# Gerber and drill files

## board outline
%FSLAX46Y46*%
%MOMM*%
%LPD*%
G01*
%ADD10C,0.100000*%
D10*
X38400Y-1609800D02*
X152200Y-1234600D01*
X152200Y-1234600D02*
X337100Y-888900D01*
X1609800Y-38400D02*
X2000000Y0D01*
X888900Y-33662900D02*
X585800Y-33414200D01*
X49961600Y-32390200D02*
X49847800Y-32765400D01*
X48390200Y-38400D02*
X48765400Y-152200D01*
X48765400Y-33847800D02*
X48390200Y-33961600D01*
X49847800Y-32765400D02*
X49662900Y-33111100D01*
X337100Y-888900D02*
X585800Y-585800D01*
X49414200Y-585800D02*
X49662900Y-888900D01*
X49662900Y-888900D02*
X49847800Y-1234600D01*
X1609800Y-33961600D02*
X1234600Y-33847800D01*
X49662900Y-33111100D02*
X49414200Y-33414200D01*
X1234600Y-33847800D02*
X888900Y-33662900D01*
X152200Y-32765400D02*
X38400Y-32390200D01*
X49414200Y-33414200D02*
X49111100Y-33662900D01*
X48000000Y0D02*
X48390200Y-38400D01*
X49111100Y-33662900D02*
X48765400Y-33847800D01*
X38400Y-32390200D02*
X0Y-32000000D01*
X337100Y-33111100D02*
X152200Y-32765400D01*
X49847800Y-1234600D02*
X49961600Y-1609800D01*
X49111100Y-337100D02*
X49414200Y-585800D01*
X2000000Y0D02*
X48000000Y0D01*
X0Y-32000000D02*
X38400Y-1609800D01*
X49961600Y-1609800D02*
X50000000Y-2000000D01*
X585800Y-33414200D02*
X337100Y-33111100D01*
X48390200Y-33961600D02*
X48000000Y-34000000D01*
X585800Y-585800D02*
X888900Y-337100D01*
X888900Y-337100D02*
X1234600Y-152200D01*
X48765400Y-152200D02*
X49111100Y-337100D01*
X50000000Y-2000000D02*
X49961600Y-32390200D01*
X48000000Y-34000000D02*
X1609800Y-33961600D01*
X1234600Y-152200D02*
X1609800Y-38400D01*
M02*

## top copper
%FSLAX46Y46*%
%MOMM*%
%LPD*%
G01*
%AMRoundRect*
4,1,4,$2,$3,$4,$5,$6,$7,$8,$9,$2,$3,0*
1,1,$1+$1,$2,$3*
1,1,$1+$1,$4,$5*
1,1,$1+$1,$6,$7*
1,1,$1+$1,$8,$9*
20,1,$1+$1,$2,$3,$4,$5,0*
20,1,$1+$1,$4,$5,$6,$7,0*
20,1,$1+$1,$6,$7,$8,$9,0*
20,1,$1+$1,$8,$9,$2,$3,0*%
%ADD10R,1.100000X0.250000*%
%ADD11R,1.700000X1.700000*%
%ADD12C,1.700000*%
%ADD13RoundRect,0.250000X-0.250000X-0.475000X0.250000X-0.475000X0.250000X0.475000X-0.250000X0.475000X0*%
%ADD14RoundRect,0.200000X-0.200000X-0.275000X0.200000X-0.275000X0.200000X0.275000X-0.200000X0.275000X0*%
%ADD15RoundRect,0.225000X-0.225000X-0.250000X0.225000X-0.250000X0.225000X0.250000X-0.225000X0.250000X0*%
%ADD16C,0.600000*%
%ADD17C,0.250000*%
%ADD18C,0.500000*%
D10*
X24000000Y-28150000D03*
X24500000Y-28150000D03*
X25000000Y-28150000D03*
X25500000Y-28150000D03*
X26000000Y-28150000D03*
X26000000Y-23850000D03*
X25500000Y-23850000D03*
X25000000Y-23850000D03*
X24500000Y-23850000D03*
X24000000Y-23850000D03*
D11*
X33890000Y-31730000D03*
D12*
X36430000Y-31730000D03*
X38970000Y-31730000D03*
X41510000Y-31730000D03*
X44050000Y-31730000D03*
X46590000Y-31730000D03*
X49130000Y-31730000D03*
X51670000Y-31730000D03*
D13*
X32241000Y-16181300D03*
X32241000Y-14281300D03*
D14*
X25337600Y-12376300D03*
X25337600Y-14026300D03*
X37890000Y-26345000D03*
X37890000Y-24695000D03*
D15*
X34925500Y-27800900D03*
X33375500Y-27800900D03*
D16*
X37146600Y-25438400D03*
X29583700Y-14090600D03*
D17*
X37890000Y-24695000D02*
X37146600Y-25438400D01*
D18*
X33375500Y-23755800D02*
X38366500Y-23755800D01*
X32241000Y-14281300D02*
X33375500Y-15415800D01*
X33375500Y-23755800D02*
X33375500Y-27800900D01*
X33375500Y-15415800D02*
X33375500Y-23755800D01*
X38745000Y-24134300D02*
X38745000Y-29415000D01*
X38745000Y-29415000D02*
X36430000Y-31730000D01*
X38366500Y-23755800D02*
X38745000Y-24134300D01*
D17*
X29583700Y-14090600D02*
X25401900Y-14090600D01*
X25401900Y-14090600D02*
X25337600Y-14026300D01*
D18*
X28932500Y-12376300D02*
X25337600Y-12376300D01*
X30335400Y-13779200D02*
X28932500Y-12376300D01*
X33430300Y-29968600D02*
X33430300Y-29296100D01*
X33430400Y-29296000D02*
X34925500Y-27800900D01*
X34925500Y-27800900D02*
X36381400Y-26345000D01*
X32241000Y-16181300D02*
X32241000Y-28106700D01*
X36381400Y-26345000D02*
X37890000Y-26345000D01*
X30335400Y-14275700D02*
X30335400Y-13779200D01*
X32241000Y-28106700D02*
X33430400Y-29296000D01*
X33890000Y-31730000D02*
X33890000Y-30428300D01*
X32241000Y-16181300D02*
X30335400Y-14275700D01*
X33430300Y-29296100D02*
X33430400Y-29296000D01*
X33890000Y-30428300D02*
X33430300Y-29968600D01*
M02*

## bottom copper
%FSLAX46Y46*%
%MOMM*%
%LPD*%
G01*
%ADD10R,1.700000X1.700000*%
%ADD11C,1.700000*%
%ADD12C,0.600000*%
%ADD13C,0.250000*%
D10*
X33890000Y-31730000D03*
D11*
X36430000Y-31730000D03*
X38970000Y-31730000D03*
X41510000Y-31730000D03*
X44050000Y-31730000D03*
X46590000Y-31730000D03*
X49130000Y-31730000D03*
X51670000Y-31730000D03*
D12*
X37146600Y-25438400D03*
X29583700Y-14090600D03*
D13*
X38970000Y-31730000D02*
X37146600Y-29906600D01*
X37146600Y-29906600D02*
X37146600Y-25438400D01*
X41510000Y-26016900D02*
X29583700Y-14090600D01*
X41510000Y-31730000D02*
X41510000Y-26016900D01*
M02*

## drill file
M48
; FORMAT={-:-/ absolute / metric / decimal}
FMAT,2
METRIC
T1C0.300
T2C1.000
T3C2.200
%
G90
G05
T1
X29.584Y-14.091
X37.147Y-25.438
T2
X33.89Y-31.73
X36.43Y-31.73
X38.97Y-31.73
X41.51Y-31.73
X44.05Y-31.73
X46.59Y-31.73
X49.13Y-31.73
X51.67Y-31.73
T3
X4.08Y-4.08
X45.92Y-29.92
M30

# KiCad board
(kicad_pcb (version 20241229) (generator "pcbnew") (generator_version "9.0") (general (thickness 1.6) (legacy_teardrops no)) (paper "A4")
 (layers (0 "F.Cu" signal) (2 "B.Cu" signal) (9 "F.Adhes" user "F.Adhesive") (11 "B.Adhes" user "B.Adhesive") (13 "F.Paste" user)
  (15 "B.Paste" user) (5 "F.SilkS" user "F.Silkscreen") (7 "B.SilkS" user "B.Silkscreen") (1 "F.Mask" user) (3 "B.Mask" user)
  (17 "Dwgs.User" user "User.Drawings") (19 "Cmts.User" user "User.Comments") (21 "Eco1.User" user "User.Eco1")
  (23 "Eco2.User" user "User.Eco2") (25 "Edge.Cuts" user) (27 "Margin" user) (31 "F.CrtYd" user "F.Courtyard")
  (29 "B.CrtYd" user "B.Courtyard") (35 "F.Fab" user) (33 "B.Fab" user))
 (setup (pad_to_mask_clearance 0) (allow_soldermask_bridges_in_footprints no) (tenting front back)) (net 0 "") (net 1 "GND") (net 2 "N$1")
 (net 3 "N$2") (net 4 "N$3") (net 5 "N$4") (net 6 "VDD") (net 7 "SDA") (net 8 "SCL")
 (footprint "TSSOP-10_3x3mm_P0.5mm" (layer "F.Cu") (at 25 26 90)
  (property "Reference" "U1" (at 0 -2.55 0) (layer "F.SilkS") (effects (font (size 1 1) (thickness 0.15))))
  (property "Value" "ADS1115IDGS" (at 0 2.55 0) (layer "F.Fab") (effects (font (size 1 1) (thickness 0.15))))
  (pad "1" smd rect (at -2.15 -1) (size 1.1 0.25) (layers "F.Cu" "F.Mask" "F.Paste") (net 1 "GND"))
  (pad "2" smd rect (at -2.15 -0.5) (size 1.1 0.25) (layers "F.Cu" "F.Mask" "F.Paste"))
  (pad "3" smd rect (at -2.15 0) (size 1.1 0.25) (layers "F.Cu" "F.Mask" "F.Paste") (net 1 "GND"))
  (pad "4" smd rect (at -2.15 0.5) (size 1.1 0.25) (layers "F.Cu" "F.Mask" "F.Paste") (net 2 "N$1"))
  (pad "5" smd rect (at -2.15 1) (size 1.1 0.25) (layers "F.Cu" "F.Mask" "F.Paste") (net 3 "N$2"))
  (pad "6" smd rect (at 2.15 1) (size 1.1 0.25) (layers "F.Cu" "F.Mask" "F.Paste") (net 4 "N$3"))
  (pad "7" smd rect (at 2.15 0.5) (size 1.1 0.25) (layers "F.Cu" "F.Mask" "F.Paste") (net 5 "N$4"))
  (pad "8" smd rect (at 2.15 0) (size 1.1 0.25) (layers "F.Cu" "F.Mask" "F.Paste") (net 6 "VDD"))
  (pad "9" smd rect (at 2.15 -0.5) (size 1.1 0.25) (layers "F.Cu" "F.Mask" "F.Paste") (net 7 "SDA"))
  (pad "10" smd rect (at 2.15 -1) (size 1.1 0.25) (layers "F.Cu" "F.Mask" "F.Paste") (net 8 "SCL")))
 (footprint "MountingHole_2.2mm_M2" (layer "F.Cu") (at 4.08 4.08)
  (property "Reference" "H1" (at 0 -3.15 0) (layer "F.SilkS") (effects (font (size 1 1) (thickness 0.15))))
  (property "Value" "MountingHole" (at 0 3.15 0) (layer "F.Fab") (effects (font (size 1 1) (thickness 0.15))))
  (pad "" np_thru_hole circle (at 0 0) (size 2.2 2.2) (drill 2.2) (layers "*.Cu" "*.Mask")))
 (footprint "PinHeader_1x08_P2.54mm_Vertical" (layer "F.Cu") (at 33.89 31.73 90)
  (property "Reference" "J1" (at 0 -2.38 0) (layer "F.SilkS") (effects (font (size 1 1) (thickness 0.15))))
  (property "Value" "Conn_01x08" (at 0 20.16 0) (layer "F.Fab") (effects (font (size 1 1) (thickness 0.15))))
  (pad "1" thru_hole rect (at 0 0) (size 1.7 1.7) (drill 1) (layers "*.Cu" "*.Mask") (remove_unused_layers no) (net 6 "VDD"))
  (pad "2" thru_hole circle (at 0 2.54) (size 1.7 1.7) (drill 1) (layers "*.Cu" "*.Mask") (remove_unused_layers no) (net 1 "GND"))
  (pad "3" thru_hole circle (at 0 5.08) (size 1.7 1.7) (drill 1) (layers "*.Cu" "*.Mask") (remove_unused_layers no) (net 7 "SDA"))
  (pad "4" thru_hole circle (at 0 7.62) (size 1.7 1.7) (drill 1) (layers "*.Cu" "*.Mask") (remove_unused_layers no) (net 8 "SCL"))
  (pad "5" thru_hole circle (at 0 10.16) (size 1.7 1.7) (drill 1) (layers "*.Cu" "*.Mask") (remove_unused_layers no) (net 2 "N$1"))
  (pad "6" thru_hole circle (at 0 12.7) (size 1.7 1.7) (drill 1) (layers "*.Cu" "*.Mask") (remove_unused_layers no) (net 3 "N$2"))
  (pad "7" thru_hole circle (at 0 15.24) (size 1.7 1.7) (drill 1) (layers "*.Cu" "*.Mask") (remove_unused_layers no) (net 4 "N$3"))
  (pad "8" thru_hole circle (at 0 17.78) (size 1.7 1.7) (drill 1) (layers "*.Cu" "*.Mask") (remove_unused_layers no) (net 5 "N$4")))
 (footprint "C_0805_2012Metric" (layer "F.Cu") (at 32.241 15.2313 90)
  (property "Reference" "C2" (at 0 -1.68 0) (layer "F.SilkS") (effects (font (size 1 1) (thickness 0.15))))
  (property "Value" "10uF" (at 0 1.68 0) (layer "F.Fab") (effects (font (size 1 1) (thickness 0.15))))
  (pad "1" smd roundrect (at -0.95 0) (size 1 1.45) (layers "F.Cu" "F.Mask" "F.Paste") (roundrect_rratio 0.25) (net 6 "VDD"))
  (pad "2" smd roundrect (at 0.95 0) (size 1 1.45) (layers "F.Cu" "F.Mask" "F.Paste") (roundrect_rratio 0.25) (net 1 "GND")))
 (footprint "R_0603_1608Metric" (layer "F.Cu") (at 25.3376 13.2013 -90)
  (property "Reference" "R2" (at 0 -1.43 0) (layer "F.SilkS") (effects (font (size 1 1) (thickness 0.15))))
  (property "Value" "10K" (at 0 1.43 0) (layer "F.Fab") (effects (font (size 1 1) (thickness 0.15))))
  (pad "1" smd roundrect (at -0.825 0) (size 0.8 0.95) (layers "F.Cu" "F.Mask" "F.Paste") (roundrect_rratio 0.25) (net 6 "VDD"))
  (pad "2" smd roundrect (at 0.825 0) (size 0.8 0.95) (layers "F.Cu" "F.Mask" "F.Paste") (roundrect_rratio 0.25) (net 8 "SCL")))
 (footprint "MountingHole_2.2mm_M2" (layer "F.Cu") (at 45.92 29.92)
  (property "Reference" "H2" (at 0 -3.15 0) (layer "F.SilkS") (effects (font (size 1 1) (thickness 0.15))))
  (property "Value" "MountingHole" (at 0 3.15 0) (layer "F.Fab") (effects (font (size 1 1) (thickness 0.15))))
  (pad "" np_thru_hole circle (at 0 0) (size 2.2 2.2) (drill 2.2) (layers "*.Cu" "*.Mask")))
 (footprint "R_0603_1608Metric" (layer "F.Cu") (at 37.89 25.52 90)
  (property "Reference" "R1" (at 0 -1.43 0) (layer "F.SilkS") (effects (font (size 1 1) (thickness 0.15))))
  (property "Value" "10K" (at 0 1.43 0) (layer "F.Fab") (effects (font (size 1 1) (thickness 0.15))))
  (pad "1" smd roundrect (at -0.825 0) (size 0.8 0.95) (layers "F.Cu" "F.Mask" "F.Paste") (roundrect_rratio 0.25) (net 6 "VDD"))
  (pad "2" smd roundrect (at 0.825 0) (size 0.8 0.95) (layers "F.Cu" "F.Mask" "F.Paste") (roundrect_rratio 0.25) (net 7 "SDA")))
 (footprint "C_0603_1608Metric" (layer "F.Cu") (at 34.1505 27.8009 180)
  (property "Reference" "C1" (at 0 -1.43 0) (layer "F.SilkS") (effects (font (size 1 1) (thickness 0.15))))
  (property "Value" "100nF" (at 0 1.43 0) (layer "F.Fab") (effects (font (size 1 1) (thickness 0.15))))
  (pad "1" smd roundrect (at -0.775 0) (size 0.9 0.95) (layers "F.Cu" "F.Mask" "F.Paste") (roundrect_rratio 0.25) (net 6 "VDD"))
  (pad "2" smd roundrect (at 0.775 0) (size 0.9 0.95) (layers "F.Cu" "F.Mask" "F.Paste") (roundrect_rratio 0.25) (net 1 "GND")))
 (gr_line (start 0.0384 1.6098) (end 0.1522 1.2346) (stroke (width 0.1) (type solid)) (layer "Edge.Cuts"))
 (gr_line (start 0.1522 1.2346) (end 0.3371 0.8889) (stroke (width 0.1) (type solid)) (layer "Edge.Cuts"))
 (gr_line (start 1.6098 0.0384) (end 2 0) (stroke (width 0.1) (type solid)) (layer "Edge.Cuts"))
 (gr_line (start 0.8889 33.6629) (end 0.5858 33.4142) (stroke (width 0.1) (type solid)) (layer "Edge.Cuts"))
 (gr_line (start 49.9616 32.3902) (end 49.8478 32.7654) (stroke (width 0.1) (type solid)) (layer "Edge.Cuts"))
 (gr_line (start 48.3902 0.0384) (end 48.7654 0.1522) (stroke (width 0.1) (type solid)) (layer "Edge.Cuts"))
 (gr_line (start 48.7654 33.8478) (end 48.3902 33.9616) (stroke (width 0.1) (type solid)) (layer "Edge.Cuts"))
 (gr_line (start 49.8478 32.7654) (end 49.6629 33.1111) (stroke (width 0.1) (type solid)) (layer "Edge.Cuts"))
 (gr_line (start 0.3371 0.8889) (end 0.5858 0.5858) (stroke (width 0.1) (type solid)) (layer "Edge.Cuts"))
 (gr_line (start 49.4142 0.5858) (end 49.6629 0.8889) (stroke (width 0.1) (type solid)) (layer "Edge.Cuts"))
 (gr_line (start 49.6629 0.8889) (end 49.8478 1.2346) (stroke (width 0.1) (type solid)) (layer "Edge.Cuts"))
 (gr_line (start 1.6098 33.9616) (end 1.2346 33.8478) (stroke (width 0.1) (type solid)) (layer "Edge.Cuts"))
 (gr_line (start 49.6629 33.1111) (end 49.4142 33.4142) (stroke (width 0.1) (type solid)) (layer "Edge.Cuts"))
 (gr_line (start 1.2346 33.8478) (end 0.8889 33.6629) (stroke (width 0.1) (type solid)) (layer "Edge.Cuts"))
 (gr_line (start 0.1522 32.7654) (end 0.0384 32.3902) (stroke (width 0.1) (type solid)) (layer "Edge.Cuts"))
 (gr_line (start 49.4142 33.4142) (end 49.1111 33.6629) (stroke (width 0.1) (type solid)) (layer "Edge.Cuts"))
 (gr_line (start 48 0) (end 48.3902 0.0384) (stroke (width 0.1) (type solid)) (layer "Edge.Cuts"))
 (gr_line (start 49.1111 33.6629) (end 48.7654 33.8478) (stroke (width 0.1) (type solid)) (layer "Edge.Cuts"))
 (gr_line (start 0.0384 32.3902) (end 0 32) (stroke (width 0.1) (type solid)) (layer "Edge.Cuts"))
 (gr_line (start 0.3371 33.1111) (end 0.1522 32.7654) (stroke (width 0.1) (type solid)) (layer "Edge.Cuts"))
 (gr_line (start 49.8478 1.2346) (end 49.9616 1.6098) (stroke (width 0.1) (type solid)) (layer "Edge.Cuts"))
 (gr_line (start 49.1111 0.3371) (end 49.4142 0.5858) (stroke (width 0.1) (type solid)) (layer "Edge.Cuts"))
 (gr_line (start 2 0) (end 48 0) (stroke (width 0.1) (type solid)) (layer "Edge.Cuts"))
 (gr_line (start 0 32) (end 0.0384 1.6098) (stroke (width 0.1) (type solid)) (layer "Edge.Cuts"))
 (gr_line (start 49.9616 1.6098) (end 50 2) (stroke (width 0.1) (type solid)) (layer "Edge.Cuts"))
 (gr_line (start 0.5858 33.4142) (end 0.3371 33.1111) (stroke (width 0.1) (type solid)) (layer "Edge.Cuts"))
 (gr_line (start 48.3902 33.9616) (end 48 34) (stroke (width 0.1) (type solid)) (layer "Edge.Cuts"))
 (gr_line (start 0.5858 0.5858) (end 0.8889 0.3371) (stroke (width 0.1) (type solid)) (layer "Edge.Cuts"))
 (gr_line (start 0.8889 0.3371) (end 1.2346 0.1522) (stroke (width 0.1) (type solid)) (layer "Edge.Cuts"))
 (gr_line (start 48.7654 0.1522) (end 49.1111 0.3371) (stroke (width 0.1) (type solid)) (layer "Edge.Cuts"))
 (gr_line (start 50 2) (end 49.9616 32.3902) (stroke (width 0.1) (type solid)) (layer "Edge.Cuts"))
 (gr_line (start 48 34) (end 1.6098 33.9616) (stroke (width 0.1) (type solid)) (layer "Edge.Cuts"))
 (gr_line (start 1.2346 0.1522) (end 1.6098 0.0384) (stroke (width 0.1) (type solid)) (layer "Edge.Cuts"))
 (segment (start 37.89 24.695) (end 37.1466 25.4384) (width 0.25) (layer "F.Cu") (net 7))
 (via (at 37.1466 25.4384) (size 0.6) (drill 0.3) (layers "F.Cu" "B.Cu") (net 7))
 (segment (start 38.97 31.73) (end 37.1466 29.9066) (width 0.25) (layer "B.Cu") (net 7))
 (segment (start 37.1466 29.9066) (end 37.1466 25.4384) (width 0.25) (layer "B.Cu") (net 7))
 (segment (start 33.3755 23.7558) (end 38.3665 23.7558) (width 0.5) (layer "F.Cu") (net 1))
 (segment (start 32.241 14.2813) (end 33.3755 15.4158) (width 0.5) (layer "F.Cu") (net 1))
 (segment (start 33.3755 23.7558) (end 33.3755 27.8009) (width 0.5) (layer "F.Cu") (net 1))
 (segment (start 33.3755 15.4158) (end 33.3755 23.7558) (width 0.5) (layer "F.Cu") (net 1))
 (segment (start 38.745 24.1343) (end 38.745 29.415) (width 0.5) (layer "F.Cu") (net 1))
 (segment (start 38.745 29.415) (end 36.43 31.73) (width 0.5) (layer "F.Cu") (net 1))
 (segment (start 38.3665 23.7558) (end 38.745 24.1343) (width 0.5) (layer "F.Cu") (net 1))
 (segment (start 29.5837 14.0906) (end 25.4019 14.0906) (width 0.25) (layer "F.Cu") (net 8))
 (segment (start 25.4019 14.0906) (end 25.3376 14.0263) (width 0.25) (layer "F.Cu") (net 8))
 (via (at 29.5837 14.0906) (size 0.6) (drill 0.3) (layers "F.Cu" "B.Cu") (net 8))
 (segment (start 41.51 26.0169) (end 29.5837 14.0906) (width 0.25) (layer "B.Cu") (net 8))
 (segment (start 41.51 31.73) (end 41.51 26.0169) (width 0.25) (layer "B.Cu") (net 8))
 (segment (start 28.9325 12.3763) (end 25.3376 12.3763) (width 0.5) (layer "F.Cu") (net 6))
 (segment (start 30.3354 13.7792) (end 28.9325 12.3763) (width 0.5) (layer "F.Cu") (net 6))
 (segment (start 33.4303 29.9686) (end 33.4303 29.2961) (width 0.5) (layer "F.Cu") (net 6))
 (segment (start 33.4304 29.296) (end 34.9255 27.8009) (width 0.5) (layer "F.Cu") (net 6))
 (segment (start 34.9255 27.8009) (end 36.3814 26.345) (width 0.5) (layer "F.Cu") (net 6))
 (segment (start 32.241 16.1813) (end 32.241 28.1067) (width 0.5) (layer "F.Cu") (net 6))
 (segment (start 36.3814 26.345) (end 37.89 26.345) (width 0.5) (layer "F.Cu") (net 6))
 (segment (start 30.3354 14.2757) (end 30.3354 13.7792) (width 0.5) (layer "F.Cu") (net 6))
 (segment (start 32.241 28.1067) (end 33.4304 29.296) (width 0.5) (layer "F.Cu") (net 6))
 (segment (start 33.89 31.73) (end 33.89 30.4283) (width 0.5) (layer "F.Cu") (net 6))
 (segment (start 32.241 16.1813) (end 30.3354 14.2757) (width 0.5) (layer "F.Cu") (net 6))
 (segment (start 33.4303 29.2961) (end 33.4304 29.296) (width 0.5) (layer "F.Cu") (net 6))
 (segment (start 33.89 30.4283) (end 33.4303 29.9686) (width 0.5) (layer "F.Cu") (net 6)))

